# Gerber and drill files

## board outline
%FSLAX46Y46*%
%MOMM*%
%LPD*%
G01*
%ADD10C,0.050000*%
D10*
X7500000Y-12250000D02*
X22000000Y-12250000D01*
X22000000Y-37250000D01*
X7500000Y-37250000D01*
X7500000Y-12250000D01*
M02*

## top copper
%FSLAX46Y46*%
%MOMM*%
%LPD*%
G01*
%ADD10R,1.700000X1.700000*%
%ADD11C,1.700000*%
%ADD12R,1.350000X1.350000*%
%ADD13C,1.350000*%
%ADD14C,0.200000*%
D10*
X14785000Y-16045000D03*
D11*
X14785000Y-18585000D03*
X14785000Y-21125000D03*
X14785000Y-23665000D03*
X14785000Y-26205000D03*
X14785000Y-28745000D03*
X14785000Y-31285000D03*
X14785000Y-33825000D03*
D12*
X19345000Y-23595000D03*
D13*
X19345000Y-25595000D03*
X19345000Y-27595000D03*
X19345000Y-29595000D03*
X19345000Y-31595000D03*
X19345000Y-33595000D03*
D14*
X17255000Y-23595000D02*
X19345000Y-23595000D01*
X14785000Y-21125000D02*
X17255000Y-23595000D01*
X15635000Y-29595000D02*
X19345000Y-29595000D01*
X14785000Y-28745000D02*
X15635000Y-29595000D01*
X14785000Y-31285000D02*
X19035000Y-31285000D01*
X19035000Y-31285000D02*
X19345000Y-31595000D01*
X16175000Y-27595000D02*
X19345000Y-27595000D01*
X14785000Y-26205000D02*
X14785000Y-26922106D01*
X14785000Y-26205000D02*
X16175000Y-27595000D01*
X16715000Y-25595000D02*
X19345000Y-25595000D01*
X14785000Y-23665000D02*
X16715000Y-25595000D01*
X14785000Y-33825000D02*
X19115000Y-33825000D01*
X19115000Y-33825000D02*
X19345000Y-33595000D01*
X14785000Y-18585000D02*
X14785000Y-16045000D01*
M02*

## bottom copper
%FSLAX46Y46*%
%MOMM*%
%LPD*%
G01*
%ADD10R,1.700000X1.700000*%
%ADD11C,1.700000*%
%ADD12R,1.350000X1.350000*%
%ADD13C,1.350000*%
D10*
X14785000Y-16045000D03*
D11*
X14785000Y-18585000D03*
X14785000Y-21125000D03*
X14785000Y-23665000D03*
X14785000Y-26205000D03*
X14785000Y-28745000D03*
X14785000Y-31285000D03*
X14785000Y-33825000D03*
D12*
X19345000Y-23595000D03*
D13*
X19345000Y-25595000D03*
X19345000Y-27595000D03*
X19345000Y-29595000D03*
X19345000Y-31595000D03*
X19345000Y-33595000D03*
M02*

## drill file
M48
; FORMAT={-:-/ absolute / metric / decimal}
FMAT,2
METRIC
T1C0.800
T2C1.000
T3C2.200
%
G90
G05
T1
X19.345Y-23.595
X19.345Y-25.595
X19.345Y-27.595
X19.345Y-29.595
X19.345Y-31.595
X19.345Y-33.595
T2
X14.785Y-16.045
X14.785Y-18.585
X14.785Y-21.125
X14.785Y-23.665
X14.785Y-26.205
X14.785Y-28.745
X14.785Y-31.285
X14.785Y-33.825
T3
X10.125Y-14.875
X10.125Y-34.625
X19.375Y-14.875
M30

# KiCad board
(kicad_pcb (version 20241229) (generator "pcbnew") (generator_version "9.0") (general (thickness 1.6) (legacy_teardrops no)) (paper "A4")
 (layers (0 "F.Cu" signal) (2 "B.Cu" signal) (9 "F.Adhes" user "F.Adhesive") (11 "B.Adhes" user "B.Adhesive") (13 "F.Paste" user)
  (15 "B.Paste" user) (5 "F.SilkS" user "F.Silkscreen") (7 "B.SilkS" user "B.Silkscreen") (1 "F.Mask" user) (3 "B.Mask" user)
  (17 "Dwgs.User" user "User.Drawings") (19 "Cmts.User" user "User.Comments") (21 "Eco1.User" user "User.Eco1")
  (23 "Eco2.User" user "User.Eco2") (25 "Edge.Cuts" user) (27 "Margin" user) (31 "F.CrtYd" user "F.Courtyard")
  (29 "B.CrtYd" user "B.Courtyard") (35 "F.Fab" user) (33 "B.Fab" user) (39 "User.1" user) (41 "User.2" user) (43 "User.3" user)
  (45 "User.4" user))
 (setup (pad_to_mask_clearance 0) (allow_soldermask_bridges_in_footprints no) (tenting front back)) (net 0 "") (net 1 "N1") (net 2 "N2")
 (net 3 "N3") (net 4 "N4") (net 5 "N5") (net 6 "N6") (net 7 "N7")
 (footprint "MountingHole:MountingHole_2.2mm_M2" (layer "F.Cu") (at 10.125 34.625)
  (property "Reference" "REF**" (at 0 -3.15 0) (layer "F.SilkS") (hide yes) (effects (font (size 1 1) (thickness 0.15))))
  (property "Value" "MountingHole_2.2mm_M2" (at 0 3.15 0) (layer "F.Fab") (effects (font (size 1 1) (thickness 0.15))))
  (pad "" np_thru_hole circle (at 0 0) (size 2.2 2.2) (drill 2.2) (layers "*.Cu" "*.Mask")))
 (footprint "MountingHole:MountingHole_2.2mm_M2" (layer "F.Cu") (at 10.125 14.875)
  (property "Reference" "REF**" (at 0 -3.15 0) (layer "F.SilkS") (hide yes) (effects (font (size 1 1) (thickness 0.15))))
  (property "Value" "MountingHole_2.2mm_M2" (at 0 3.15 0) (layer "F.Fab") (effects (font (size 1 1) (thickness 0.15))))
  (pad "" np_thru_hole circle (at 0 0) (size 2.2 2.2) (drill 2.2) (layers "*.Cu" "*.Mask")))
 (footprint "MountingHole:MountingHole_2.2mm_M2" (layer "F.Cu") (at 19.375 14.875)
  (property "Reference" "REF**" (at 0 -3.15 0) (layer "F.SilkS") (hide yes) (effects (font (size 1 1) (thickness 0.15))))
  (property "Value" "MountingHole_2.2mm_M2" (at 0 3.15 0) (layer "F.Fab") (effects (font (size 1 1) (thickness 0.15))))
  (pad "" np_thru_hole circle (at 0 0) (size 2.2 2.2) (drill 2.2) (layers "*.Cu" "*.Mask")))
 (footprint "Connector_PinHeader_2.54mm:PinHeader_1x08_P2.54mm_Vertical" (layer "F.Cu") (at 14.785 16.045)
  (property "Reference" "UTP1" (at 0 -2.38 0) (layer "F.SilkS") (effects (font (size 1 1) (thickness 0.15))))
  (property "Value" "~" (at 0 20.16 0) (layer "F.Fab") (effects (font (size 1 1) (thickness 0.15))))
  (pad "1" thru_hole rect (at 0 0) (size 1.7 1.7) (drill 1) (layers "*.Cu" "*.Mask") (remove_unused_layers no) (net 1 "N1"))
  (pad "2" thru_hole circle (at 0 2.54) (size 1.7 1.7) (drill 1) (layers "*.Cu" "*.Mask") (remove_unused_layers no) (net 1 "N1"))
  (pad "3" thru_hole circle (at 0 5.08) (size 1.7 1.7) (drill 1) (layers "*.Cu" "*.Mask") (remove_unused_layers no) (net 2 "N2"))
  (pad "4" thru_hole circle (at 0 7.62) (size 1.7 1.7) (drill 1) (layers "*.Cu" "*.Mask") (remove_unused_layers no) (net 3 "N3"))
  (pad "5" thru_hole circle (at 0 10.16) (size 1.7 1.7) (drill 1) (layers "*.Cu" "*.Mask") (remove_unused_layers no) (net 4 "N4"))
  (pad "6" thru_hole circle (at 0 12.7) (size 1.7 1.7) (drill 1) (layers "*.Cu" "*.Mask") (remove_unused_layers no) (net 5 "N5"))
  (pad "7" thru_hole circle (at 0 15.24) (size 1.7 1.7) (drill 1) (layers "*.Cu" "*.Mask") (remove_unused_layers no) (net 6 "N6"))
  (pad "8" thru_hole circle (at 0 17.78) (size 1.7 1.7) (drill 1) (layers "*.Cu" "*.Mask") (remove_unused_layers no) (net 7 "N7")))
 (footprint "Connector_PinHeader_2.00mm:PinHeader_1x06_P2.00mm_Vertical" (layer "B.Cu") (at 19.345 23.595 180)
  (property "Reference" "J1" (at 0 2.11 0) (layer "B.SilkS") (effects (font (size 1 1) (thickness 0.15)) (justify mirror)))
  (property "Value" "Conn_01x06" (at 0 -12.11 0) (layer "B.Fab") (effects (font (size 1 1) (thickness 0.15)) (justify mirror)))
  (pad "1" thru_hole rect (at 0 0 180) (size 1.35 1.35) (drill 0.8) (layers "*.Cu" "*.Mask") (remove_unused_layers no) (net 2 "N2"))
  (pad "2" thru_hole circle (at 0 -2 180) (size 1.35 1.35) (drill 0.8) (layers "*.Cu" "*.Mask") (remove_unused_layers no) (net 3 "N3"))
  (pad "3" thru_hole circle (at 0 -4 180) (size 1.35 1.35) (drill 0.8) (layers "*.Cu" "*.Mask") (remove_unused_layers no) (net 4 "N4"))
  (pad "4" thru_hole circle (at 0 -6 180) (size 1.35 1.35) (drill 0.8) (layers "*.Cu" "*.Mask") (remove_unused_layers no) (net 5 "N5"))
  (pad "5" thru_hole circle (at 0 -8 180) (size 1.35 1.35) (drill 0.8) (layers "*.Cu" "*.Mask") (remove_unused_layers no) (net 6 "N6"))
  (pad "6" thru_hole circle (at 0 -10 180) (size 1.35 1.35) (drill 0.8) (layers "*.Cu" "*.Mask") (remove_unused_layers no) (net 7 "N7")))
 (gr_rect (start 7.5 12.25) (end 22 37.25) (stroke (width 0.05) (type default)) (fill no) (layer "Edge.Cuts"))
 (segment (start 17.255 23.595) (end 19.345 23.595) (width 0.2) (layer "F.Cu") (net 2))
 (segment (start 14.785 21.125) (end 17.255 23.595) (width 0.2) (layer "F.Cu") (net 2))
 (segment (start 15.635 29.595) (end 19.345 29.595) (width 0.2) (layer "F.Cu") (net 5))
 (segment (start 14.785 28.745) (end 15.635 29.595) (width 0.2) (layer "F.Cu") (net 5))
 (segment (start 14.785 31.285) (end 19.035 31.285) (width 0.2) (layer "F.Cu") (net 6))
 (segment (start 19.035 31.285) (end 19.345 31.595) (width 0.2) (layer "F.Cu") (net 6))
 (segment (start 16.175 27.595) (end 19.345 27.595) (width 0.2) (layer "F.Cu") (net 4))
 (segment (start 14.785 26.205) (end 14.785 26.922106) (width 0.2) (layer "F.Cu") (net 4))
 (segment (start 14.785 26.205) (end 16.175 27.595) (width 0.2) (layer "F.Cu") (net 4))
 (segment (start 16.715 25.595) (end 19.345 25.595) (width 0.2) (layer "F.Cu") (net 3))
 (segment (start 14.785 23.665) (end 16.715 25.595) (width 0.2) (layer "F.Cu") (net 3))
 (segment (start 14.785 33.825) (end 19.115 33.825) (width 0.2) (layer "F.Cu") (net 7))
 (segment (start 19.115 33.825) (end 19.345 33.595) (width 0.2) (layer "F.Cu") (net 7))
 (segment (start 14.785 18.585) (end 14.785 16.045) (width 0.2) (layer "F.Cu") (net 1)))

